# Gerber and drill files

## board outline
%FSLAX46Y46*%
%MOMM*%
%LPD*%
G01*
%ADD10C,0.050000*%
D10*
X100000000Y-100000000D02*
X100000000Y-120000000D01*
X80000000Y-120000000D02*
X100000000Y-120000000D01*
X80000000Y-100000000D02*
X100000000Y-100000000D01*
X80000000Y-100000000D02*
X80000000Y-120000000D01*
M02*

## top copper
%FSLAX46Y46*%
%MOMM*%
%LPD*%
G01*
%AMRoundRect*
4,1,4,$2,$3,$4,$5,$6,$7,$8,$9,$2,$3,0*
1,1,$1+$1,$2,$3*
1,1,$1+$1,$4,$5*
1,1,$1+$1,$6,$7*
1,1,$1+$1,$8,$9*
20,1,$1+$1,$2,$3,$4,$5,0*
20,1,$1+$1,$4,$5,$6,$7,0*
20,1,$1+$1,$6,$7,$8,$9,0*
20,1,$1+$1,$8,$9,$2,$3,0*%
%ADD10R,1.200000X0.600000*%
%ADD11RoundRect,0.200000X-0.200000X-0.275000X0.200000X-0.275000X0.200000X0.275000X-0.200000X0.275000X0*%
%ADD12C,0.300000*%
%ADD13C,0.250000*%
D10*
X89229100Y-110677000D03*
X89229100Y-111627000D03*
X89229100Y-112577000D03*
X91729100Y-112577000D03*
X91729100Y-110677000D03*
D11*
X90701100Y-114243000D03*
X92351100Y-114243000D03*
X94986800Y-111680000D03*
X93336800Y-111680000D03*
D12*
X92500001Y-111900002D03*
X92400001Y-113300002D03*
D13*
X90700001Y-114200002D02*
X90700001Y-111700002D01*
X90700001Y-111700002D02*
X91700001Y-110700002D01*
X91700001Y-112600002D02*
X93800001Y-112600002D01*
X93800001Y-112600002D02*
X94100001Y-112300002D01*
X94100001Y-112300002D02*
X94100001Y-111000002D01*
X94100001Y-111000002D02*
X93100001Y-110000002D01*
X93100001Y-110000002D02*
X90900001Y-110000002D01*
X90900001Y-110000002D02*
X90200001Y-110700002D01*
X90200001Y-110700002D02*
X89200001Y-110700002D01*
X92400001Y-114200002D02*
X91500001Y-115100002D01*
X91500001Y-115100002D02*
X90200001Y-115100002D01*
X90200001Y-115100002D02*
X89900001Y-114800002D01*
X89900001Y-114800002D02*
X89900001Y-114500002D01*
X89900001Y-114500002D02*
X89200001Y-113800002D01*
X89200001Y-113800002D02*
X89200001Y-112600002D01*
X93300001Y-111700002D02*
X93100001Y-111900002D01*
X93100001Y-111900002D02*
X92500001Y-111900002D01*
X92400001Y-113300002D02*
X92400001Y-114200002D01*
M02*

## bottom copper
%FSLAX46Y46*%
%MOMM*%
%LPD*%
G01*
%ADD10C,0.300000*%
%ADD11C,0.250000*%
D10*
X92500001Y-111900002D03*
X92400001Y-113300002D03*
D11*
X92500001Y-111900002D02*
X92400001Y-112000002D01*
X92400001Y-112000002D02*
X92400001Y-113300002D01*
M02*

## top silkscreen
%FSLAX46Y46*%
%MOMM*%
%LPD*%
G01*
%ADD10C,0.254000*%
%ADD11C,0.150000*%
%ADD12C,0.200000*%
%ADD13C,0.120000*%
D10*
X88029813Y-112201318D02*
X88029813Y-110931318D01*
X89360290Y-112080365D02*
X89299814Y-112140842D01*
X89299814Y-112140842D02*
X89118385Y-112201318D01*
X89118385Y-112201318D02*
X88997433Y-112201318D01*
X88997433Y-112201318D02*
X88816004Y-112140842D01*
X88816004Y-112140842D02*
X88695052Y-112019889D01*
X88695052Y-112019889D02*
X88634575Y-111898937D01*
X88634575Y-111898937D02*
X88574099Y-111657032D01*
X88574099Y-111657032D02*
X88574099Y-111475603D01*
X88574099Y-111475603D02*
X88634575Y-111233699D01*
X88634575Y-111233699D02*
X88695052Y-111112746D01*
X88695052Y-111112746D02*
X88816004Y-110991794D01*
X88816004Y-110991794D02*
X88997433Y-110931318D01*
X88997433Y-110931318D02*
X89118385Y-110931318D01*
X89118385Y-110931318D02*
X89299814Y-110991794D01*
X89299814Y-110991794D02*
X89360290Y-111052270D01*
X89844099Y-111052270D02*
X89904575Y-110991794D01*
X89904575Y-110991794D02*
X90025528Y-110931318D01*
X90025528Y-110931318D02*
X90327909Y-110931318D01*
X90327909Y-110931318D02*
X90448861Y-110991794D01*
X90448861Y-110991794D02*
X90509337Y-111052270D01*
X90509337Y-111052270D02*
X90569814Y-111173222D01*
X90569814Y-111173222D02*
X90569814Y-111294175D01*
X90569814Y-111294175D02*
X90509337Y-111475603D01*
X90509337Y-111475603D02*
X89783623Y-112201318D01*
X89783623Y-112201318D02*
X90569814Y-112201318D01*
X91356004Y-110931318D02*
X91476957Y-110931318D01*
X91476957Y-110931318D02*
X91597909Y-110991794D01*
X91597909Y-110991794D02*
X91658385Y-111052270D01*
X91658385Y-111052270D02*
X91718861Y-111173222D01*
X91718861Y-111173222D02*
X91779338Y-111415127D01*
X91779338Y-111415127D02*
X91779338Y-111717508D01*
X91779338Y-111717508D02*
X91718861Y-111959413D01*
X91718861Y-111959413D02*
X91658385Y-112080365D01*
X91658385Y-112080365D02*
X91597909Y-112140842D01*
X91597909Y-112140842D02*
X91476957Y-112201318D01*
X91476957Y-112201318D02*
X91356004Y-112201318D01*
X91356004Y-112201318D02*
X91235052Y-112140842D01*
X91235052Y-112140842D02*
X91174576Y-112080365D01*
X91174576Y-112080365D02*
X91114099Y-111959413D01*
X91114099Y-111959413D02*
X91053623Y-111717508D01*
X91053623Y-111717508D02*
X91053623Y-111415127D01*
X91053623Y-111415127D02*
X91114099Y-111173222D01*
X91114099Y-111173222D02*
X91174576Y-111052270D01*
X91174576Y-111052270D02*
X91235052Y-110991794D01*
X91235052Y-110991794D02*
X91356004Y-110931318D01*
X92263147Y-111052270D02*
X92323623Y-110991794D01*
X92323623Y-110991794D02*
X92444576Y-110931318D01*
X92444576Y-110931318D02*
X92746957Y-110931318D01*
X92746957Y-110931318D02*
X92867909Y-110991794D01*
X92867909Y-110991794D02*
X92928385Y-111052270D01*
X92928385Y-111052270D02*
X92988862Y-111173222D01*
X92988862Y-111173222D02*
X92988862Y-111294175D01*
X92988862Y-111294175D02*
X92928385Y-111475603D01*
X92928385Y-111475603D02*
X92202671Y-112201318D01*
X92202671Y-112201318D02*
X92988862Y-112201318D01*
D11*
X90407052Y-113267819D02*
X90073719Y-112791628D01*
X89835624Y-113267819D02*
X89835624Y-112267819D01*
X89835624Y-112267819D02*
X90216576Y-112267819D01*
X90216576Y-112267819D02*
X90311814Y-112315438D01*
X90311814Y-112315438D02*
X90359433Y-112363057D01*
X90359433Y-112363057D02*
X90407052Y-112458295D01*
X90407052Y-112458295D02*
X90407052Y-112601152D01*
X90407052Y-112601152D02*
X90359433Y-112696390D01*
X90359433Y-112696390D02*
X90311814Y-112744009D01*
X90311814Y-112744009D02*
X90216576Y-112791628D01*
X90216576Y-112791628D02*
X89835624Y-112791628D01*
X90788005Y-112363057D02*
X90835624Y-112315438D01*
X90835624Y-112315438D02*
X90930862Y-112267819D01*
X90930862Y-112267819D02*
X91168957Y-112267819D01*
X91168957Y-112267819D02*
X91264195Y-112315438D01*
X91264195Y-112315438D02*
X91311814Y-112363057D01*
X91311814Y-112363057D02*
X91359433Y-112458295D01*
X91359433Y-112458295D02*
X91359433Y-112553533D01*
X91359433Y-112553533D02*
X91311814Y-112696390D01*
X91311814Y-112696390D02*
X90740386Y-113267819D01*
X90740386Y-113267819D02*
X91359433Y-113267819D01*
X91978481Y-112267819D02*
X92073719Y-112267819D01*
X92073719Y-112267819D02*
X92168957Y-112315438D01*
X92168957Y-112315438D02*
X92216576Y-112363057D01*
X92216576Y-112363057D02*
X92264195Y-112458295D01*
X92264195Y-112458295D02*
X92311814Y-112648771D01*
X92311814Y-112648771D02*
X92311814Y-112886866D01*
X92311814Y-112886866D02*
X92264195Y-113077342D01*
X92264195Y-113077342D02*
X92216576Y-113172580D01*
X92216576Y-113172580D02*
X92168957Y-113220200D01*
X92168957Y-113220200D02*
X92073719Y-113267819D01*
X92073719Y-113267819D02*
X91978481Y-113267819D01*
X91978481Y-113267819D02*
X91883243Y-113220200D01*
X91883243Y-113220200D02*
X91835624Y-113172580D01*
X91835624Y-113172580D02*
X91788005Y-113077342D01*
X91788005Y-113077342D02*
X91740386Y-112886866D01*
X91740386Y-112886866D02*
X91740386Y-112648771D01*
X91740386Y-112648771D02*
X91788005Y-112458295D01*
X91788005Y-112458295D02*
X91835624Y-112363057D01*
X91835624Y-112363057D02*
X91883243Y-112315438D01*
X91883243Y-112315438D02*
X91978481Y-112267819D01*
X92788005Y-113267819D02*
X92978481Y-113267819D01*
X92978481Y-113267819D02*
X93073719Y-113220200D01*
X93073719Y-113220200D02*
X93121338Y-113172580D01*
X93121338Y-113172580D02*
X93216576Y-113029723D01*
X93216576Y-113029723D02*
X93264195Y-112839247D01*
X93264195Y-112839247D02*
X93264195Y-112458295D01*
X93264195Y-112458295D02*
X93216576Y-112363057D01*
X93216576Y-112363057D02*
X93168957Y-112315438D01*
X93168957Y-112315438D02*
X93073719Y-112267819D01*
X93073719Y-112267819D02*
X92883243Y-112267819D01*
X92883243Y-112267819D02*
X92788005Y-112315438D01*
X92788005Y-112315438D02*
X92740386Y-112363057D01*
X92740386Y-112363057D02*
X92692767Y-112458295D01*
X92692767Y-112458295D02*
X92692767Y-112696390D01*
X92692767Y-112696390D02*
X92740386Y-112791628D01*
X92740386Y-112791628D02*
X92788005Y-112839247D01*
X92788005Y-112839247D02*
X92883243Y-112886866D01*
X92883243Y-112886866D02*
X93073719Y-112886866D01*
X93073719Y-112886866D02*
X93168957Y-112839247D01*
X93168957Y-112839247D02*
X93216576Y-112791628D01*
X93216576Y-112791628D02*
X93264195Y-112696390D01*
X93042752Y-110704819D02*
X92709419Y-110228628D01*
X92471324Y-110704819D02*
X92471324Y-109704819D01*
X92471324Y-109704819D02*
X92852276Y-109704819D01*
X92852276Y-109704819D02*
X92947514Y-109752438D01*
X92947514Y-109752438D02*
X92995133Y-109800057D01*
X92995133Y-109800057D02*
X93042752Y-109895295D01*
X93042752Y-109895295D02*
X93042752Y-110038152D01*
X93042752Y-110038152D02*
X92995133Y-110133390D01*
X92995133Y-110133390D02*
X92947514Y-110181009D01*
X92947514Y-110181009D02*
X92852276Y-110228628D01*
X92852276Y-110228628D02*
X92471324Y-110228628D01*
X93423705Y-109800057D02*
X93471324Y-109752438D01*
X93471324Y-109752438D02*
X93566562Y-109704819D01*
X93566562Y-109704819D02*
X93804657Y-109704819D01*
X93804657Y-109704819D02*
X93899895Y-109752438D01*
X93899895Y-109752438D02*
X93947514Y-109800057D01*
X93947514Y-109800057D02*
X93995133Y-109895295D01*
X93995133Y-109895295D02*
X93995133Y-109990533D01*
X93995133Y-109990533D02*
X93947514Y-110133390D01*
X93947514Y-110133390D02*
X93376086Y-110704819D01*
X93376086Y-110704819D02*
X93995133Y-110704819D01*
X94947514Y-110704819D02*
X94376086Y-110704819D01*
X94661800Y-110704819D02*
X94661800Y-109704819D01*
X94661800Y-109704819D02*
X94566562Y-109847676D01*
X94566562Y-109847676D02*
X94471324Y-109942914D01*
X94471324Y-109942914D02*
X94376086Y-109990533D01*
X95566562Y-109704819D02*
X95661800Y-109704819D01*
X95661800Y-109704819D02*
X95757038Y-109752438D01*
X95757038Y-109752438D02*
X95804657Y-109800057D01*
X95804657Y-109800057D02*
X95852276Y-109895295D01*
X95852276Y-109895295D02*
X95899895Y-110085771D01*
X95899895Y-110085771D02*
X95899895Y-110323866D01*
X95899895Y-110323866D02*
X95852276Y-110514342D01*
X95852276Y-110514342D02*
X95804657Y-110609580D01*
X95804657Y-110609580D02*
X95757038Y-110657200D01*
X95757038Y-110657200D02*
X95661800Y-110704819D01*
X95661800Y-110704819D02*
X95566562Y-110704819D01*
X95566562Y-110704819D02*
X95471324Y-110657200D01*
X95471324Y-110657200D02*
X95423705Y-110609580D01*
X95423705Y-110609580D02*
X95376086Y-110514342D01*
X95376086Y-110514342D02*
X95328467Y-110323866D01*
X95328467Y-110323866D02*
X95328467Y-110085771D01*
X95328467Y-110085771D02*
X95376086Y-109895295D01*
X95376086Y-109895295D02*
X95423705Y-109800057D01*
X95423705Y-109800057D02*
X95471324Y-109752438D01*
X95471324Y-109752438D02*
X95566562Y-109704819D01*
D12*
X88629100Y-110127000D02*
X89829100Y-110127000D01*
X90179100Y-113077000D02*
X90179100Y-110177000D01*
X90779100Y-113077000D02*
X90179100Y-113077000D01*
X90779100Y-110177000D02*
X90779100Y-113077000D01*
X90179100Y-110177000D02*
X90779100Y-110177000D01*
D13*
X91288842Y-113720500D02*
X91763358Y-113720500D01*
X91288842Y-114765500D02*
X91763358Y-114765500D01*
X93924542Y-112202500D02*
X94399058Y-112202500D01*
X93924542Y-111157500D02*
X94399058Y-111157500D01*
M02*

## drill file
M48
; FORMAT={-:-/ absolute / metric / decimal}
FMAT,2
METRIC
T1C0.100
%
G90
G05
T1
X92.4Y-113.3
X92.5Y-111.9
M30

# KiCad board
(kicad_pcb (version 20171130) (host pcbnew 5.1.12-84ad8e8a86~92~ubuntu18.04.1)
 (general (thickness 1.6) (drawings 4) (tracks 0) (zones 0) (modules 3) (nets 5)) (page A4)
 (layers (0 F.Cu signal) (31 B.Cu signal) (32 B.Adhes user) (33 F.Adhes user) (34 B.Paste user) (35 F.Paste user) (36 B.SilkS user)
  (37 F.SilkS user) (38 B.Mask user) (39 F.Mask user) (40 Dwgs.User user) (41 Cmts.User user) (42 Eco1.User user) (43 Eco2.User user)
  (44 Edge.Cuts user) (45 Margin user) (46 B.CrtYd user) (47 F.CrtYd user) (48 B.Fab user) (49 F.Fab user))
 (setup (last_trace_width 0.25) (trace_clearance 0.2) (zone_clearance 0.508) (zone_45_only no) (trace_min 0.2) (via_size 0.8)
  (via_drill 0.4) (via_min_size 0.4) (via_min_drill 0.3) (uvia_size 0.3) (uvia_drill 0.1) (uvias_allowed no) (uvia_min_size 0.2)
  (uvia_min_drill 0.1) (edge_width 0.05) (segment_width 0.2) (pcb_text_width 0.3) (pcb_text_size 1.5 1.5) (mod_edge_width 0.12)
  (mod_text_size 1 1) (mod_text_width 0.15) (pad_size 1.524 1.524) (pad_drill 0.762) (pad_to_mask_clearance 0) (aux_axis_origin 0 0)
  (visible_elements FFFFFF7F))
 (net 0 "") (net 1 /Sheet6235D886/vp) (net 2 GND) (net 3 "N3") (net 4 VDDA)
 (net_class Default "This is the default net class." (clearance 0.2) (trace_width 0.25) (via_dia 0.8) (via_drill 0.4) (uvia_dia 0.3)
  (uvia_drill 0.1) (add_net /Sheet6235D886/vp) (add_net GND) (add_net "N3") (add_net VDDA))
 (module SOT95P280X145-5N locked (layer F.Cu) (at 90.479100 111.627000)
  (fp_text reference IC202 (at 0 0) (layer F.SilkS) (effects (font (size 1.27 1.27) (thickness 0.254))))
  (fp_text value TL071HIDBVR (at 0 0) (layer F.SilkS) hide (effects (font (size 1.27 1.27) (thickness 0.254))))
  (fp_line (start -1.85 -1.5) (end -0.65 -1.5) (layer F.SilkS) (width 0.2))
  (fp_line (start -0.3 1.45) (end -0.3 -1.45) (layer F.SilkS) (width 0.2))
  (fp_line (start 0.3 1.45) (end -0.3 1.45) (layer F.SilkS) (width 0.2))
  (fp_line (start 0.3 -1.45) (end 0.3 1.45) (layer F.SilkS) (width 0.2))
  (fp_line (start -0.3 -1.45) (end 0.3 -1.45) (layer F.SilkS) (width 0.2))
  (pad 1 smd rect (at -1.25 -0.95 90.000000) (size 0.6 1.2) (layers F.Cu F.Mask F.Paste) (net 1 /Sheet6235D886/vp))
  (pad 2 smd rect (at -1.25 0 90.000000) (size 0.6 1.2) (layers F.Cu F.Mask F.Paste) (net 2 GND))
  (pad 3 smd rect (at -1.25 0.95 90.000000) (size 0.6 1.2) (layers F.Cu F.Mask F.Paste) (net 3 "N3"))
  (pad 4 smd rect (at 1.25 0.95 90.000000) (size 0.6 1.2) (layers F.Cu F.Mask F.Paste) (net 1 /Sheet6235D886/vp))
  (pad 5 smd rect (at 1.25 -0.95 90.000000) (size 0.6 1.2) (layers F.Cu F.Mask F.Paste) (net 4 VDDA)))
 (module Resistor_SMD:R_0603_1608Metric (layer F.Cu) (at 91.526100 114.243000)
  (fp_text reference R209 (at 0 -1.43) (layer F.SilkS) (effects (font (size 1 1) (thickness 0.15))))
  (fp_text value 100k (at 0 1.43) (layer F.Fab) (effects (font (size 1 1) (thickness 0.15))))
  (fp_line (start -0.237258 -0.5225) (end 0.237258 -0.5225) (layer F.SilkS) (width 0.12))
  (fp_line (start -0.237258 0.5225) (end 0.237258 0.5225) (layer F.SilkS) (width 0.12))
  (pad 1 smd roundrect (at -0.825 0) (size 0.8 0.95) (layers F.Cu F.Mask F.Paste) (roundrect_rratio 0.25) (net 4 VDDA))
  (pad 2 smd roundrect (at 0.825 0) (size 0.8 0.95) (layers F.Cu F.Mask F.Paste) (roundrect_rratio 0.25) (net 3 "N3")))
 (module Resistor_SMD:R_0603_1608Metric (layer F.Cu) (at 94.161800 111.680000)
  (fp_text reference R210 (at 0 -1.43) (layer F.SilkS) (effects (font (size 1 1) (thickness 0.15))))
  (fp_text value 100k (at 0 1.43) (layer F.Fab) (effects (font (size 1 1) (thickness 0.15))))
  (fp_line (start -0.237258 0.5225) (end 0.237258 0.5225) (layer F.SilkS) (width 0.12))
  (fp_line (start -0.237258 -0.5225) (end 0.237258 -0.5225) (layer F.SilkS) (width 0.12))
  (pad 2 smd roundrect (at 0.825 0) (size 0.8 0.95) (layers F.Cu F.Mask F.Paste) (roundrect_rratio 0.25) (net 2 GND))
  (pad 1 smd roundrect (at -0.825 0) (size 0.8 0.95) (layers F.Cu F.Mask F.Paste) (roundrect_rratio 0.25) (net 3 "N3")))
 (gr_line (start 100 100) (end 100 120) (layer Edge.Cuts) (width 0.05))
 (gr_line (start 80 120) (end 100 120) (layer Edge.Cuts) (width 0.05))
 (gr_line (start 80 100) (end 100 100) (layer Edge.Cuts) (width 0.05))
 (gr_line (start 80 100) (end 80 120) (layer Edge.Cuts) (width 0.05))
 (segment (start 90.700001 114.200002) (end 90.700001 111.700002) (width 0.250000) (layer F.Cu) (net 4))
 (segment (start 90.700001 111.700002) (end 91.700001 110.700002) (width 0.250000) (layer F.Cu) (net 4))
 (segment (start 91.700001 112.600002) (end 93.800001 112.600002) (width 0.250000) (layer F.Cu) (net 1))
 (segment (start 93.800001 112.600002) (end 94.100001 112.300002) (width 0.250000) (layer F.Cu) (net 1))
 (segment (start 94.100001 112.300002) (end 94.100001 111.000002) (width 0.250000) (layer F.Cu) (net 1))
 (segment (start 94.100001 111.000002) (end 93.100001 110.000002) (width 0.250000) (layer F.Cu) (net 1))
 (segment (start 93.100001 110.000002) (end 90.900001 110.000002) (width 0.250000) (layer F.Cu) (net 1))
 (segment (start 90.900001 110.000002) (end 90.200001 110.700002) (width 0.250000) (layer F.Cu) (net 1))
 (segment (start 90.200001 110.700002) (end 89.200001 110.700002) (width 0.250000) (layer F.Cu) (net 1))
 (segment (start 92.400001 114.200002) (end 91.500001 115.100002) (width 0.250000) (layer F.Cu) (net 3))
 (segment (start 91.500001 115.100002) (end 90.200001 115.100002) (width 0.250000) (layer F.Cu) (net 3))
 (segment (start 90.200001 115.100002) (end 89.900001 114.800002) (width 0.250000) (layer F.Cu) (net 3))
 (segment (start 89.900001 114.800002) (end 89.900001 114.500002) (width 0.250000) (layer F.Cu) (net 3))
 (segment (start 89.900001 114.500002) (end 89.200001 113.800002) (width 0.250000) (layer F.Cu) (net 3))
 (segment (start 89.200001 113.800002) (end 89.200001 112.600002) (width 0.250000) (layer F.Cu) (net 3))
 (segment (start 93.300001 111.700002) (end 93.100001 111.900002) (width 0.250000) (layer F.Cu) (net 3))
 (segment (start 93.100001 111.900002) (end 92.500001 111.900002) (width 0.250000) (layer F.Cu) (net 3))
 (segment (start 92.500001 111.900002) (end 92.400001 112.000002) (width 0.250000) (layer B.Cu) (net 3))
 (segment (start 92.400001 112.000002) (end 92.400001 113.300002) (width 0.250000) (layer B.Cu) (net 3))
 (segment (start 92.400001 113.300002) (end 92.400001 114.200002) (width 0.250000) (layer F.Cu) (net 3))
 (via micro (at 92.500001 111.900002) (size 0.300000) (drill 0.100000) (layers F.Cu B.Cu) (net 3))
 (via micro (at 92.400001 113.300002) (size 0.300000) (drill 0.100000) (layers F.Cu B.Cu) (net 3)))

